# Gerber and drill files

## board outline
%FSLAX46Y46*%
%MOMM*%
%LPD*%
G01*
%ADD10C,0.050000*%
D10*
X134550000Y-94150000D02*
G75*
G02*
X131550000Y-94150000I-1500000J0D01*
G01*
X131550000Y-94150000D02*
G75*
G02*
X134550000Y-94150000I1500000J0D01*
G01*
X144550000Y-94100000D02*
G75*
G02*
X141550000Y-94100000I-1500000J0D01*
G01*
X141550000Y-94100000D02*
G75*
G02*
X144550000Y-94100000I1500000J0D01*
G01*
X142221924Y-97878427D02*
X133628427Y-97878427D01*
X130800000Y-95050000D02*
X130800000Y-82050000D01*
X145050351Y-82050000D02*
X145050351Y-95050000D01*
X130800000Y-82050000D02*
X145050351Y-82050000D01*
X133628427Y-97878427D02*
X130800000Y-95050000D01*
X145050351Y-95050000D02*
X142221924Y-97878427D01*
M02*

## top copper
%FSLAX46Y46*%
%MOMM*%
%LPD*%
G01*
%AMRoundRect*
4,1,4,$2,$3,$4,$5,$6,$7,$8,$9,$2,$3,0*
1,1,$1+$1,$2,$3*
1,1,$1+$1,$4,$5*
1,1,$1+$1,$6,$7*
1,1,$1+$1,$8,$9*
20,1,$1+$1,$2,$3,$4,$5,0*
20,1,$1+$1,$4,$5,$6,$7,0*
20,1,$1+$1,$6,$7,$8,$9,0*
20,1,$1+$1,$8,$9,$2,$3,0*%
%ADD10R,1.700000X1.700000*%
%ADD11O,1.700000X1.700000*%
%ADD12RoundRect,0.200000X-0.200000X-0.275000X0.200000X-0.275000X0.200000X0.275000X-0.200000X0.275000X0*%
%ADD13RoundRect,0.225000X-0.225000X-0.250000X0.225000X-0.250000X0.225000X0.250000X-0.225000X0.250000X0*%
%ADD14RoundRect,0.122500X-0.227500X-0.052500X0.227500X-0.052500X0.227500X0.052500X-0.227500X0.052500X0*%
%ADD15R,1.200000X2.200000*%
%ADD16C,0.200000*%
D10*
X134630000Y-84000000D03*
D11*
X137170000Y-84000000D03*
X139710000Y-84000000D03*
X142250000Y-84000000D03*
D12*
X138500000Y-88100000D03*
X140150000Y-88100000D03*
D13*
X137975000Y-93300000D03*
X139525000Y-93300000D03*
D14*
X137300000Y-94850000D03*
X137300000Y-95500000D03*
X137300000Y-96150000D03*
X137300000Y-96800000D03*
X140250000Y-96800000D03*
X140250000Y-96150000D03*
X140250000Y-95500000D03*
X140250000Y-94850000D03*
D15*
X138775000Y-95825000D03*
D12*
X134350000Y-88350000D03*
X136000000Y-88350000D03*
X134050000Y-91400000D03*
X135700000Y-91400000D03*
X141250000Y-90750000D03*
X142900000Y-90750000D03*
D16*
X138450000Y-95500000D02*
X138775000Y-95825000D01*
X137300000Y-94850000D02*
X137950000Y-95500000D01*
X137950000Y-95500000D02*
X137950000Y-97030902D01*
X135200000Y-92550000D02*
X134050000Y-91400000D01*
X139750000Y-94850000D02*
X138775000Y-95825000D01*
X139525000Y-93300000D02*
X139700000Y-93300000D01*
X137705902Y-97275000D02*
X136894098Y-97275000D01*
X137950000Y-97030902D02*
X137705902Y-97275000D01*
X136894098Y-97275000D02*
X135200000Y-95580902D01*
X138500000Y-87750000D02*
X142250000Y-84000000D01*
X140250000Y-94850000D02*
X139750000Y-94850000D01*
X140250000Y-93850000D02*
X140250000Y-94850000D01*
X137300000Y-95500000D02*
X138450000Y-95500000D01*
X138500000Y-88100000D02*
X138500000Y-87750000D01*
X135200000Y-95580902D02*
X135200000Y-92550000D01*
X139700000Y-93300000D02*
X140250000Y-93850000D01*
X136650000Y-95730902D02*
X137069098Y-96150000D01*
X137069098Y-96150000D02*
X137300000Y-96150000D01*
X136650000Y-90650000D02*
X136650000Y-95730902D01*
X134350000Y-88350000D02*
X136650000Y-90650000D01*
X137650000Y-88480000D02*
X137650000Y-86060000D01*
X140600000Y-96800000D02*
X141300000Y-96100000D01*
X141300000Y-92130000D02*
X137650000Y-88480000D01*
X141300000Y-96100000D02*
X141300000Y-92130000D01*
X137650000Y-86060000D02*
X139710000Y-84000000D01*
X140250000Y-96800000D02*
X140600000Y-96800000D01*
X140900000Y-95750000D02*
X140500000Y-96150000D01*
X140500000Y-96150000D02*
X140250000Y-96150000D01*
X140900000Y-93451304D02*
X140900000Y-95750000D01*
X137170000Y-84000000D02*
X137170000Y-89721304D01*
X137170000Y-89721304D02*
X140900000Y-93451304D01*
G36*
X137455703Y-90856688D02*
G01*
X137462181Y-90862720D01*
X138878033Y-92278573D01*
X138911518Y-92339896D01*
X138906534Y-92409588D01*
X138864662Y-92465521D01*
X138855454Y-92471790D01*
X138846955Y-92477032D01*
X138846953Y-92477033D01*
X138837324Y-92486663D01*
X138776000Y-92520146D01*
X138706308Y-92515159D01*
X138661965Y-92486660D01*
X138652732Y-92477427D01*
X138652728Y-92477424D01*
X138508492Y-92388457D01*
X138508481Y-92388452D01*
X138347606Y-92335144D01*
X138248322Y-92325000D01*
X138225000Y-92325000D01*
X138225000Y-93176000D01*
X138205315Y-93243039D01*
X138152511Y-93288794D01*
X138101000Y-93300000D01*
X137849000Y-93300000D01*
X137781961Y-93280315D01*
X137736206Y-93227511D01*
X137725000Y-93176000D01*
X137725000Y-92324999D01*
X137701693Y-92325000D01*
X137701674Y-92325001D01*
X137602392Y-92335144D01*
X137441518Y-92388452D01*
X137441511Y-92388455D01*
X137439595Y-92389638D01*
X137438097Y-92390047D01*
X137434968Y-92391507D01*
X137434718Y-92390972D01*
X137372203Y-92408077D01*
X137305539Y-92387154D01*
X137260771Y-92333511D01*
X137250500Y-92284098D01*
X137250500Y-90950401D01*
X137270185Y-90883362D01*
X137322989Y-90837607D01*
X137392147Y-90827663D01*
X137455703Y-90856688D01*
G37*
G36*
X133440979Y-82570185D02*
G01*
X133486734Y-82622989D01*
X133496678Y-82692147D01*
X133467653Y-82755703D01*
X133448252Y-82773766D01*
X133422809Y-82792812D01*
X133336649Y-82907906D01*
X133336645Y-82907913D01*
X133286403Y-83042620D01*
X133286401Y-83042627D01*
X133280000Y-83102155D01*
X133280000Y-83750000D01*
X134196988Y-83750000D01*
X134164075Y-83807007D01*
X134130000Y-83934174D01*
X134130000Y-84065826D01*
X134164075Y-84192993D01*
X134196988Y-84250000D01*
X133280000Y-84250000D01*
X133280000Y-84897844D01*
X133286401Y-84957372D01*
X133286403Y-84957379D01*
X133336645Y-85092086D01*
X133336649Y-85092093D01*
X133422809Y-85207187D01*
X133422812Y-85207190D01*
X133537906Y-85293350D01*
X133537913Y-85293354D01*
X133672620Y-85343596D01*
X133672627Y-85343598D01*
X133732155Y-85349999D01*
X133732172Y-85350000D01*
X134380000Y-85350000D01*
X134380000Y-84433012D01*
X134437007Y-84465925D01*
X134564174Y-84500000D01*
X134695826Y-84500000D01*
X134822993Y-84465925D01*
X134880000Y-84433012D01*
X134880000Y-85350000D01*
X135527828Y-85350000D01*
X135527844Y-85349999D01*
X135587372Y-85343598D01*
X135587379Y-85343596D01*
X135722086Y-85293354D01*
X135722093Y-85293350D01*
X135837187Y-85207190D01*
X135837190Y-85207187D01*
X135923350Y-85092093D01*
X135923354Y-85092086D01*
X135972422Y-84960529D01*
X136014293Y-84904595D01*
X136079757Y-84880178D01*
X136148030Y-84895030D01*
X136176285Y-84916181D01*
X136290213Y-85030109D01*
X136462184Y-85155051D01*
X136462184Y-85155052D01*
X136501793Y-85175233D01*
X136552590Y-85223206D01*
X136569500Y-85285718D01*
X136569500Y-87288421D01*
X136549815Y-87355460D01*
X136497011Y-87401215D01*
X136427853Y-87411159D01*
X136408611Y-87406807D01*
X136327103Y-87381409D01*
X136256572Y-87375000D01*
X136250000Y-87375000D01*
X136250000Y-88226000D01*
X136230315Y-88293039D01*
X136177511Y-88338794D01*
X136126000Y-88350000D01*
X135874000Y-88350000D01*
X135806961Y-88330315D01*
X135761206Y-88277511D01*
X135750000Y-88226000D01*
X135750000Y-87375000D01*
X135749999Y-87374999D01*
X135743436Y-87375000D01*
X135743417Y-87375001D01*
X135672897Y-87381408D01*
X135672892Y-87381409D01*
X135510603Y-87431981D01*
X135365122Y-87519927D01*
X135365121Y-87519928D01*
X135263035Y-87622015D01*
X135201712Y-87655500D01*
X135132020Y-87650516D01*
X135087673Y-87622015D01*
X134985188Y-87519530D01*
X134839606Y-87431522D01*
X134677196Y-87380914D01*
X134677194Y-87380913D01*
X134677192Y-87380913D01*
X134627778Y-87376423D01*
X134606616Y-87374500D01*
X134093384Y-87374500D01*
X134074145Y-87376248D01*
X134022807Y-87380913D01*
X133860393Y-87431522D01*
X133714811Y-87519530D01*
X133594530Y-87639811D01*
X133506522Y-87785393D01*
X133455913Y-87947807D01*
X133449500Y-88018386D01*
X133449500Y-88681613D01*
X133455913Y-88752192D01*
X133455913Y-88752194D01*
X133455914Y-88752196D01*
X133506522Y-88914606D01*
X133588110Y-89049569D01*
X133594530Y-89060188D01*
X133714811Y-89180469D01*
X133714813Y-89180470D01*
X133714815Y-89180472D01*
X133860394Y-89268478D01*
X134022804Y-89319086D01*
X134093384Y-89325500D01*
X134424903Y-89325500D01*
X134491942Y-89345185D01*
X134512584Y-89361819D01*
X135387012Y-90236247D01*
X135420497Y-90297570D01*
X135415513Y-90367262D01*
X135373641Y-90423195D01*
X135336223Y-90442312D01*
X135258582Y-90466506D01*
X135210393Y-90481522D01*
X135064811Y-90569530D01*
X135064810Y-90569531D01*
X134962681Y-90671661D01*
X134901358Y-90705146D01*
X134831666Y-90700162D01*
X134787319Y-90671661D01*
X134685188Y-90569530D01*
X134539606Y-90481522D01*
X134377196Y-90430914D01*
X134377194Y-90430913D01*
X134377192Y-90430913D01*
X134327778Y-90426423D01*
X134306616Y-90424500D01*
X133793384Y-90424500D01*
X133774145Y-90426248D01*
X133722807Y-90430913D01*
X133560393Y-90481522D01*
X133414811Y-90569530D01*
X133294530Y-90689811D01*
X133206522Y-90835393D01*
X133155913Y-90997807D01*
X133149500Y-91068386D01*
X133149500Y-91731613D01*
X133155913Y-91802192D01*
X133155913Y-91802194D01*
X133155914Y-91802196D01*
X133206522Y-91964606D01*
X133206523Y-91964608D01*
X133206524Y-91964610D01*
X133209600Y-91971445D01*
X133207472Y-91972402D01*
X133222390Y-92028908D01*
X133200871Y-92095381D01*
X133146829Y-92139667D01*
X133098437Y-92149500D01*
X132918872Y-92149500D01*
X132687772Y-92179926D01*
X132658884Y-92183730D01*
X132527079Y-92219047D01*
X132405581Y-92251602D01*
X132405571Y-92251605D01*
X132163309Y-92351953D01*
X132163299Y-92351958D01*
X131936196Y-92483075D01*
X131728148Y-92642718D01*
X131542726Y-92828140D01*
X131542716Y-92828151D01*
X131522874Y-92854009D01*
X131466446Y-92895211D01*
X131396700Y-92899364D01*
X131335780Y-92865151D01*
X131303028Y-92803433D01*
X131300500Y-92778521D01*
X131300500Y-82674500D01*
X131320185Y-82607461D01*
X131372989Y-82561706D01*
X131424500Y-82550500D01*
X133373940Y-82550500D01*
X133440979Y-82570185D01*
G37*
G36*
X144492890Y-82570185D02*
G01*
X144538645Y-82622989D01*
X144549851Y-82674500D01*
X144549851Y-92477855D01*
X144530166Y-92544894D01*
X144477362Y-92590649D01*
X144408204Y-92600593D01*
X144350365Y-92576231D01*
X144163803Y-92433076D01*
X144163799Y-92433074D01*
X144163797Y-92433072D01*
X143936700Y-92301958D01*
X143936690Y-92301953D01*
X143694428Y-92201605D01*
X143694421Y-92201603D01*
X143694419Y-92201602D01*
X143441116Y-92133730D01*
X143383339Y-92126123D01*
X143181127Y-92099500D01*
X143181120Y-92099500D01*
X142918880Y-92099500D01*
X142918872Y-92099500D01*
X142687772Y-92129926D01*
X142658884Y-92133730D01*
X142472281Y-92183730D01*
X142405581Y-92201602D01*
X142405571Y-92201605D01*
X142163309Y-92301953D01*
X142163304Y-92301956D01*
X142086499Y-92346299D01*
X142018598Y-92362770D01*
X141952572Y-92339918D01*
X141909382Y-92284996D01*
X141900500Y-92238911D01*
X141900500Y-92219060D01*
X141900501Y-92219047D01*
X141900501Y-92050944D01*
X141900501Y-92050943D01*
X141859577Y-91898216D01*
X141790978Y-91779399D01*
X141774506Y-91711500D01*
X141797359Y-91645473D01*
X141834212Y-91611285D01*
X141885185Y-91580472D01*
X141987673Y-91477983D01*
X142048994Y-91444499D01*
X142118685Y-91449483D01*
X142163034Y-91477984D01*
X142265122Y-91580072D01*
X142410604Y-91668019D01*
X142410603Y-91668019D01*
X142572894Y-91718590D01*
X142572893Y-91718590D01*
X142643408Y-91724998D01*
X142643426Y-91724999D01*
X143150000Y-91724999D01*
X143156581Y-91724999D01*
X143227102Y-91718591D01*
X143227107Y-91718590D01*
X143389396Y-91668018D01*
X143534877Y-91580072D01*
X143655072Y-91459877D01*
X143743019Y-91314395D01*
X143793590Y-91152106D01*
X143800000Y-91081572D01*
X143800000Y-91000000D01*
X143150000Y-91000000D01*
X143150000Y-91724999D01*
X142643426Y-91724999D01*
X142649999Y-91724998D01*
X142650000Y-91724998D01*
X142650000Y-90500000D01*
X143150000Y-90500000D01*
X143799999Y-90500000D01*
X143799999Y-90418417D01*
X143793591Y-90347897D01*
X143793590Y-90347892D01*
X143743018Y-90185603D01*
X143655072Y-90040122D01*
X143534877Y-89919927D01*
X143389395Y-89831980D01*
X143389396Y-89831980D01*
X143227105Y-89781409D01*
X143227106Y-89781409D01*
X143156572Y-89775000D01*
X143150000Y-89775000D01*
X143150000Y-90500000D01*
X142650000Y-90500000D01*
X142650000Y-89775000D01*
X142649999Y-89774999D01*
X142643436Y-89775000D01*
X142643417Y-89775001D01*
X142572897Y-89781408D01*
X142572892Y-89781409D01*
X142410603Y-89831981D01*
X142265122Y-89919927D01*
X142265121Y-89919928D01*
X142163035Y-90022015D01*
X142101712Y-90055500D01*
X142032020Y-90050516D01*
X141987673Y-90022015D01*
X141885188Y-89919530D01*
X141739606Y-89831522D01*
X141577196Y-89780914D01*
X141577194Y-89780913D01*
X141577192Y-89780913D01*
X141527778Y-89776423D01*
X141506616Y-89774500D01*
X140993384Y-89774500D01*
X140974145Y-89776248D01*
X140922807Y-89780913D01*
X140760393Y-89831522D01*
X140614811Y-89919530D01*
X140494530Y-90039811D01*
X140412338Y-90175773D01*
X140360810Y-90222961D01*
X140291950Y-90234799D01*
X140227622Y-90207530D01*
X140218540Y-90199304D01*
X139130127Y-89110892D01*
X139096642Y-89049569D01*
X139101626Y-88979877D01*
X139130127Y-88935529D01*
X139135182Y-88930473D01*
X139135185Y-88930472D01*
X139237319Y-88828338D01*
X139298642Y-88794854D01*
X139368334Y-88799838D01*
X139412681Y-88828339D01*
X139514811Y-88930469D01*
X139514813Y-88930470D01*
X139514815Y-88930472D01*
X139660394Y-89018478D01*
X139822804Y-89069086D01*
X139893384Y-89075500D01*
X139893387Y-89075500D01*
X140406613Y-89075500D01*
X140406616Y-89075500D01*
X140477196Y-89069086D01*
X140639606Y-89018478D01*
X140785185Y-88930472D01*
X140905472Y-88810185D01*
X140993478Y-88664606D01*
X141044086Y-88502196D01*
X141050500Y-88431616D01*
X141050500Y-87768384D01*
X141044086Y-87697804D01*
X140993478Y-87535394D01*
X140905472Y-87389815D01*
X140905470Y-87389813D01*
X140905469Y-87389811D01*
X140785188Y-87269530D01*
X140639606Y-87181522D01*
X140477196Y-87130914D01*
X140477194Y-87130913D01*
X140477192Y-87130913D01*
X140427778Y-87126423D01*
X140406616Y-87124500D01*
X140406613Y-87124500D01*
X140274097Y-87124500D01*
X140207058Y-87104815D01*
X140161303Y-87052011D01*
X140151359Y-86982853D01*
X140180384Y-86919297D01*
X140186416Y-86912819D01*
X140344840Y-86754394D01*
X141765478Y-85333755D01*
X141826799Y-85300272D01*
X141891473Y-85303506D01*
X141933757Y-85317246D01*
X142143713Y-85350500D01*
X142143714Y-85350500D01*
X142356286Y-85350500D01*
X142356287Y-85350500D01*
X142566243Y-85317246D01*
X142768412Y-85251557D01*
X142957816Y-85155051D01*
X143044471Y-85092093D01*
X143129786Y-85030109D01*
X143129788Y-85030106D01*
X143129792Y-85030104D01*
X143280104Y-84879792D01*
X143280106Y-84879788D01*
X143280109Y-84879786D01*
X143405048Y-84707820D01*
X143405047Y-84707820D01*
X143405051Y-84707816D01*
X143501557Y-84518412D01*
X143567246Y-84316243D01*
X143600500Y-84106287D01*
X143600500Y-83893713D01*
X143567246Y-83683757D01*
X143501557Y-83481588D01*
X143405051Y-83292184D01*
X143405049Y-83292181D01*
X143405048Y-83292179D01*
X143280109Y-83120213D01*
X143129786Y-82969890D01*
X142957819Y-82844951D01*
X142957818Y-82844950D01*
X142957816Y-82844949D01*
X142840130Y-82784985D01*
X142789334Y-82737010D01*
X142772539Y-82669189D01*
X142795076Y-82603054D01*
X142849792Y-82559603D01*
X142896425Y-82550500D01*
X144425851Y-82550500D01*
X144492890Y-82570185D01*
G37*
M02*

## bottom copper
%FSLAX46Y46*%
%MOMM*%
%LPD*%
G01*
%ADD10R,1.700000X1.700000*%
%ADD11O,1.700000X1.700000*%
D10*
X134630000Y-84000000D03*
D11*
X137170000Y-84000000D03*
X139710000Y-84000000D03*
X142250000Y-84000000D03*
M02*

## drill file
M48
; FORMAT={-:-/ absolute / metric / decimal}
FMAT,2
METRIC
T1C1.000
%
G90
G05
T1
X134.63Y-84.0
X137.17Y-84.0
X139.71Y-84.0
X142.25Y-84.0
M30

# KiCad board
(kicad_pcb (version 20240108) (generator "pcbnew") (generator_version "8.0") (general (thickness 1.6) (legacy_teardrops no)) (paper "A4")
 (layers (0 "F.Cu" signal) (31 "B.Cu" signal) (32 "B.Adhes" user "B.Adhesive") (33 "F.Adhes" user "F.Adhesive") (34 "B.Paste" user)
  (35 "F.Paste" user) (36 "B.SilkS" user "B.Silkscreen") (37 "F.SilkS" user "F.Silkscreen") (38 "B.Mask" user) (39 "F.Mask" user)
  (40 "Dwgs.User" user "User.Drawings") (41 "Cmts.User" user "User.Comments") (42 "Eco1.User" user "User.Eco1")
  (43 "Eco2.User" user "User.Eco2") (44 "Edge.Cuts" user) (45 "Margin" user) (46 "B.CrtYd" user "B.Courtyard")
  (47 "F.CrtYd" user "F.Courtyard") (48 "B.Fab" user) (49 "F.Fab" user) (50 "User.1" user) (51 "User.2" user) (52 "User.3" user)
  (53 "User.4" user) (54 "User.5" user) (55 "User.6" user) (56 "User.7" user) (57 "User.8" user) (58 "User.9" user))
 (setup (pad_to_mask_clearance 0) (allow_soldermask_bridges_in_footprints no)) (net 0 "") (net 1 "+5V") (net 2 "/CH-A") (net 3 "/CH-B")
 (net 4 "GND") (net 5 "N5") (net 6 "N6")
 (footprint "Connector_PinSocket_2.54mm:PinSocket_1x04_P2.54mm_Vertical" (layer "F.Cu") (at 134.63 84 90)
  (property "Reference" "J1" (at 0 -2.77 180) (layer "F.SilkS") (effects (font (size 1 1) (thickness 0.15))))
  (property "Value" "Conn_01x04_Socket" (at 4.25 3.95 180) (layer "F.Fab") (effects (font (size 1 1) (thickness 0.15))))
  (pad "1" thru_hole rect (at 0 0 90) (size 1.7 1.7) (drill 1) (layers "*.Cu" "*.Mask") (remove_unused_layers no) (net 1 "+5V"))
  (pad "2" thru_hole oval (at 0 2.54 90) (size 1.7 1.7) (drill 1) (layers "*.Cu" "*.Mask") (remove_unused_layers no) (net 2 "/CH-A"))
  (pad "3" thru_hole oval (at 0 5.08 90) (size 1.7 1.7) (drill 1) (layers "*.Cu" "*.Mask") (remove_unused_layers no) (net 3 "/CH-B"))
  (pad "4" thru_hole oval (at 0 7.62 90) (size 1.7 1.7) (drill 1) (layers "*.Cu" "*.Mask") (remove_unused_layers no) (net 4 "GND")))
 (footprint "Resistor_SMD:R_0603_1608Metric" (layer "F.Cu") (at 139.325 88.1)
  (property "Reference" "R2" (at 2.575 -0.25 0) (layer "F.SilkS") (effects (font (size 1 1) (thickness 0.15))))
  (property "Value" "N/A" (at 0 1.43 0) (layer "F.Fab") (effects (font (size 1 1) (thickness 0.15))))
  (pad "1" smd roundrect (at -0.825 0) (size 0.8 0.95) (layers "F.Cu" "F.Paste" "F.Mask") (roundrect_rratio 0.25) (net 4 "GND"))
  (pad "2" smd roundrect (at 0.825 0) (size 0.8 0.95) (layers "F.Cu" "F.Paste" "F.Mask") (roundrect_rratio 0.25) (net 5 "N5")))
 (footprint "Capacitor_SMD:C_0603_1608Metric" (layer "F.Cu") (at 138.75 93.3)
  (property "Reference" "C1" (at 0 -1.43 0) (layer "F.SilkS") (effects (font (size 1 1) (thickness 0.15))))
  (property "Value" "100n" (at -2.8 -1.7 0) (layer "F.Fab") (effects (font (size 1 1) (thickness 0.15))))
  (pad "1" smd roundrect (at -0.775 0) (size 0.9 0.95) (layers "F.Cu" "F.Paste" "F.Mask") (roundrect_rratio 0.25) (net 1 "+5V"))
  (pad "2" smd roundrect (at 0.775 0) (size 0.9 0.95) (layers "F.Cu" "F.Paste" "F.Mask") (roundrect_rratio 0.25) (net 4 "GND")))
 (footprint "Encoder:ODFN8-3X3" (layer "F.Cu") (at 138.775 95.825)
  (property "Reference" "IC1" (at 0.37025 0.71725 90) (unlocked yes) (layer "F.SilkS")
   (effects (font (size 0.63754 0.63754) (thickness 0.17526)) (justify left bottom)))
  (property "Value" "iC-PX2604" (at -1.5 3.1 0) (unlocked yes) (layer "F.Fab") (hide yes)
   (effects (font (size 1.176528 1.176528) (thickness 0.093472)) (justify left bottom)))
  (pad "1" smd roundrect (at -1.475 -0.975) (size 0.7 0.35) (layers "F.Cu" "F.Paste" "F.Mask") (roundrect_rratio 0.35) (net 4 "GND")
   (solder_mask_margin 0.075) (thermal_bridge_angle 0))
  (pad "2" smd roundrect (at -1.475 -0.325) (size 0.7 0.35) (layers "F.Cu" "F.Paste" "F.Mask") (roundrect_rratio 0.35) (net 4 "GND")
   (solder_mask_margin 0.075) (thermal_bridge_angle 0))
  (pad "3" smd roundrect (at -1.475 0.325) (size 0.7 0.35) (layers "F.Cu" "F.Paste" "F.Mask") (roundrect_rratio 0.35) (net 5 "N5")
   (solder_mask_margin 0.075) (thermal_bridge_angle 0))
  (pad "4" smd roundrect (at -1.475 0.975) (size 0.7 0.35) (layers "F.Cu" "F.Paste" "F.Mask") (roundrect_rratio 0.35) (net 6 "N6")
   (solder_mask_margin 0.075) (thermal_bridge_angle 0))
  (pad "5" smd roundrect (at 1.475 0.975) (size 0.7 0.35) (layers "F.Cu" "F.Paste" "F.Mask") (roundrect_rratio 0.35) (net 3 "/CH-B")
   (solder_mask_margin 0.075) (thermal_bridge_angle 0))
  (pad "6" smd roundrect (at 1.475 0.325) (size 0.7 0.35) (layers "F.Cu" "F.Paste" "F.Mask") (roundrect_rratio 0.35) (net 2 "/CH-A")
   (solder_mask_margin 0.075) (thermal_bridge_angle 0))
  (pad "7" smd roundrect (at 1.475 -0.325) (size 0.7 0.35) (layers "F.Cu" "F.Paste" "F.Mask") (roundrect_rratio 0.35) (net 1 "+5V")
   (solder_mask_margin 0.075) (thermal_bridge_angle 0))
  (pad "8" smd roundrect (at 1.475 -0.975) (size 0.7 0.35) (layers "F.Cu" "F.Paste" "F.Mask") (roundrect_rratio 0.35) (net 4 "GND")
   (solder_mask_margin 0.075) (thermal_bridge_angle 0))
  (pad "BP" smd rect (at 0 0) (size 1.2 2.2) (layers "F.Cu" "F.Mask") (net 4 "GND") (solder_mask_margin 0.075) (thermal_bridge_angle 0)))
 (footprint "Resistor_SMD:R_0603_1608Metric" (layer "F.Cu") (at 135.175 88.35)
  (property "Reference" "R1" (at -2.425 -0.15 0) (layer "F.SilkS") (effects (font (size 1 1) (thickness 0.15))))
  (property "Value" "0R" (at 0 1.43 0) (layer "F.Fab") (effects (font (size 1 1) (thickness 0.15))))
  (pad "1" smd roundrect (at -0.825 0) (size 0.8 0.95) (layers "F.Cu" "F.Paste" "F.Mask") (roundrect_rratio 0.25) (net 5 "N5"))
  (pad "2" smd roundrect (at 0.825 0) (size 0.8 0.95) (layers "F.Cu" "F.Paste" "F.Mask") (roundrect_rratio 0.25) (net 1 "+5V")))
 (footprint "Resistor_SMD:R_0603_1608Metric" (layer "F.Cu") (at 134.875 91.4)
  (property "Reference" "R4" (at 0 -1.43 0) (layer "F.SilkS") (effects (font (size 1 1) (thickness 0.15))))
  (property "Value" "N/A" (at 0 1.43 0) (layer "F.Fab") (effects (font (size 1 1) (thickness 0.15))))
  (pad "1" smd roundrect (at -0.825 0) (size 0.8 0.95) (layers "F.Cu" "F.Paste" "F.Mask") (roundrect_rratio 0.25) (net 4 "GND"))
  (pad "2" smd roundrect (at 0.825 0) (size 0.8 0.95) (layers "F.Cu" "F.Paste" "F.Mask") (roundrect_rratio 0.25) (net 6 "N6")))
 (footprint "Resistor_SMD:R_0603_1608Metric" (layer "F.Cu") (at 142.075 90.75)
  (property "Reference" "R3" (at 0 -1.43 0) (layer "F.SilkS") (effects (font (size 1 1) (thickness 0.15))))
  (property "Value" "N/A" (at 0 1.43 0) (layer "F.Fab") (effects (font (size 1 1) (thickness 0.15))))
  (pad "1" smd roundrect (at -0.825 0) (size 0.8 0.95) (layers "F.Cu" "F.Paste" "F.Mask") (roundrect_rratio 0.25) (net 6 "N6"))
  (pad "2" smd roundrect (at 0.825 0) (size 0.8 0.95) (layers "F.Cu" "F.Paste" "F.Mask") (roundrect_rratio 0.25) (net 1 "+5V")))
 (gr_circle (center 133.05 94.15) (end 134.55 94.15) (stroke (width 0.05) (type default)) (fill none) (layer "Edge.Cuts"))
 (gr_circle (center 143.05 94.1) (end 144.55 94.1) (stroke (width 0.05) (type default)) (fill none) (layer "Edge.Cuts"))
 (gr_line (start 142.221924 97.878427) (end 133.628427 97.878427) (stroke (width 0.05) (type default)) (layer "Edge.Cuts"))
 (gr_line (start 130.8 95.05) (end 130.8 82.05) (stroke (width 0.05) (type default)) (layer "Edge.Cuts"))
 (gr_line (start 145.050351 82.05) (end 145.050351 95.05) (stroke (width 0.05) (type default)) (layer "Edge.Cuts"))
 (gr_line (start 130.8 82.05) (end 145.050351 82.05) (stroke (width 0.05) (type default)) (layer "Edge.Cuts"))
 (gr_line (start 133.628427 97.878427) (end 130.8 95.05) (stroke (width 0.05) (type default)) (layer "Edge.Cuts"))
 (gr_line (start 145.050351 95.05) (end 142.221924 97.878427) (stroke (width 0.05) (type default)) (layer "Edge.Cuts"))
 (segment (start 138.45 95.5) (end 138.775 95.825) (width 0.2) (layer "F.Cu") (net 4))
 (segment (start 137.3 94.85) (end 137.95 95.5) (width 0.2) (layer "F.Cu") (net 4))
 (segment (start 137.95 95.5) (end 137.95 97.030902) (width 0.2) (layer "F.Cu") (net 4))
 (segment (start 135.2 92.55) (end 134.05 91.4) (width 0.2) (layer "F.Cu") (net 4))
 (segment (start 139.75 94.85) (end 138.775 95.825) (width 0.2) (layer "F.Cu") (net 4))
 (segment (start 139.525 93.3) (end 139.7 93.3) (width 0.2) (layer "F.Cu") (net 4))
 (segment (start 137.705902 97.275) (end 136.894098 97.275) (width 0.2) (layer "F.Cu") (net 4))
 (segment (start 137.95 97.030902) (end 137.705902 97.275) (width 0.2) (layer "F.Cu") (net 4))
 (segment (start 136.894098 97.275) (end 135.2 95.580902) (width 0.2) (layer "F.Cu") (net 4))
 (segment (start 138.5 87.75) (end 142.25 84) (width 0.2) (layer "F.Cu") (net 4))
 (segment (start 140.25 94.85) (end 139.75 94.85) (width 0.2) (layer "F.Cu") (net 4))
 (segment (start 140.25 93.85) (end 140.25 94.85) (width 0.2) (layer "F.Cu") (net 4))
 (segment (start 137.3 95.5) (end 138.45 95.5) (width 0.2) (layer "F.Cu") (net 4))
 (segment (start 138.5 88.1) (end 138.5 87.75) (width 0.2) (layer "F.Cu") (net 4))
 (segment (start 135.2 95.580902) (end 135.2 92.55) (width 0.2) (layer "F.Cu") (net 4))
 (segment (start 139.7 93.3) (end 140.25 93.85) (width 0.2) (layer "F.Cu") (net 4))
 (segment (start 136.65 95.730902) (end 137.069098 96.15) (width 0.2) (layer "F.Cu") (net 5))
 (segment (start 137.069098 96.15) (end 137.3 96.15) (width 0.2) (layer "F.Cu") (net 5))
 (segment (start 136.65 90.65) (end 136.65 95.730902) (width 0.2) (layer "F.Cu") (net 5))
 (segment (start 134.35 88.35) (end 136.65 90.65) (width 0.2) (layer "F.Cu") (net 5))
 (segment (start 137.65 88.48) (end 137.65 86.06) (width 0.2) (layer "F.Cu") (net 3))
 (segment (start 140.6 96.8) (end 141.3 96.1) (width 0.2) (layer "F.Cu") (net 3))
 (segment (start 141.3 92.13) (end 137.65 88.48) (width 0.2) (layer "F.Cu") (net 3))
 (segment (start 141.3 96.1) (end 141.3 92.13) (width 0.2) (layer "F.Cu") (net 3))
 (segment (start 137.65 86.06) (end 139.71 84) (width 0.2) (layer "F.Cu") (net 3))
 (segment (start 140.25 96.8) (end 140.6 96.8) (width 0.2) (layer "F.Cu") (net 3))
 (segment (start 140.9 95.75) (end 140.5 96.15) (width 0.2) (layer "F.Cu") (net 2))
 (segment (start 140.5 96.15) (end 140.25 96.15) (width 0.2) (layer "F.Cu") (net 2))
 (segment (start 140.9 93.451304) (end 140.9 95.75) (width 0.2) (layer "F.Cu") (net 2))
 (segment (start 137.17 84) (end 137.17 89.721304) (width 0.2) (layer "F.Cu") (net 2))
 (segment (start 137.17 89.721304) (end 140.9 93.451304) (width 0.2) (layer "F.Cu") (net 2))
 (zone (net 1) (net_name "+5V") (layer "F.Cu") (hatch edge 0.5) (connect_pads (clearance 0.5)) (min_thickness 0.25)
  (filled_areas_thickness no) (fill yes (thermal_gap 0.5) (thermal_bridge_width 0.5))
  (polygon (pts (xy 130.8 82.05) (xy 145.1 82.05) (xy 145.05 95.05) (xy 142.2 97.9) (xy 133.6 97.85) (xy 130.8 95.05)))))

